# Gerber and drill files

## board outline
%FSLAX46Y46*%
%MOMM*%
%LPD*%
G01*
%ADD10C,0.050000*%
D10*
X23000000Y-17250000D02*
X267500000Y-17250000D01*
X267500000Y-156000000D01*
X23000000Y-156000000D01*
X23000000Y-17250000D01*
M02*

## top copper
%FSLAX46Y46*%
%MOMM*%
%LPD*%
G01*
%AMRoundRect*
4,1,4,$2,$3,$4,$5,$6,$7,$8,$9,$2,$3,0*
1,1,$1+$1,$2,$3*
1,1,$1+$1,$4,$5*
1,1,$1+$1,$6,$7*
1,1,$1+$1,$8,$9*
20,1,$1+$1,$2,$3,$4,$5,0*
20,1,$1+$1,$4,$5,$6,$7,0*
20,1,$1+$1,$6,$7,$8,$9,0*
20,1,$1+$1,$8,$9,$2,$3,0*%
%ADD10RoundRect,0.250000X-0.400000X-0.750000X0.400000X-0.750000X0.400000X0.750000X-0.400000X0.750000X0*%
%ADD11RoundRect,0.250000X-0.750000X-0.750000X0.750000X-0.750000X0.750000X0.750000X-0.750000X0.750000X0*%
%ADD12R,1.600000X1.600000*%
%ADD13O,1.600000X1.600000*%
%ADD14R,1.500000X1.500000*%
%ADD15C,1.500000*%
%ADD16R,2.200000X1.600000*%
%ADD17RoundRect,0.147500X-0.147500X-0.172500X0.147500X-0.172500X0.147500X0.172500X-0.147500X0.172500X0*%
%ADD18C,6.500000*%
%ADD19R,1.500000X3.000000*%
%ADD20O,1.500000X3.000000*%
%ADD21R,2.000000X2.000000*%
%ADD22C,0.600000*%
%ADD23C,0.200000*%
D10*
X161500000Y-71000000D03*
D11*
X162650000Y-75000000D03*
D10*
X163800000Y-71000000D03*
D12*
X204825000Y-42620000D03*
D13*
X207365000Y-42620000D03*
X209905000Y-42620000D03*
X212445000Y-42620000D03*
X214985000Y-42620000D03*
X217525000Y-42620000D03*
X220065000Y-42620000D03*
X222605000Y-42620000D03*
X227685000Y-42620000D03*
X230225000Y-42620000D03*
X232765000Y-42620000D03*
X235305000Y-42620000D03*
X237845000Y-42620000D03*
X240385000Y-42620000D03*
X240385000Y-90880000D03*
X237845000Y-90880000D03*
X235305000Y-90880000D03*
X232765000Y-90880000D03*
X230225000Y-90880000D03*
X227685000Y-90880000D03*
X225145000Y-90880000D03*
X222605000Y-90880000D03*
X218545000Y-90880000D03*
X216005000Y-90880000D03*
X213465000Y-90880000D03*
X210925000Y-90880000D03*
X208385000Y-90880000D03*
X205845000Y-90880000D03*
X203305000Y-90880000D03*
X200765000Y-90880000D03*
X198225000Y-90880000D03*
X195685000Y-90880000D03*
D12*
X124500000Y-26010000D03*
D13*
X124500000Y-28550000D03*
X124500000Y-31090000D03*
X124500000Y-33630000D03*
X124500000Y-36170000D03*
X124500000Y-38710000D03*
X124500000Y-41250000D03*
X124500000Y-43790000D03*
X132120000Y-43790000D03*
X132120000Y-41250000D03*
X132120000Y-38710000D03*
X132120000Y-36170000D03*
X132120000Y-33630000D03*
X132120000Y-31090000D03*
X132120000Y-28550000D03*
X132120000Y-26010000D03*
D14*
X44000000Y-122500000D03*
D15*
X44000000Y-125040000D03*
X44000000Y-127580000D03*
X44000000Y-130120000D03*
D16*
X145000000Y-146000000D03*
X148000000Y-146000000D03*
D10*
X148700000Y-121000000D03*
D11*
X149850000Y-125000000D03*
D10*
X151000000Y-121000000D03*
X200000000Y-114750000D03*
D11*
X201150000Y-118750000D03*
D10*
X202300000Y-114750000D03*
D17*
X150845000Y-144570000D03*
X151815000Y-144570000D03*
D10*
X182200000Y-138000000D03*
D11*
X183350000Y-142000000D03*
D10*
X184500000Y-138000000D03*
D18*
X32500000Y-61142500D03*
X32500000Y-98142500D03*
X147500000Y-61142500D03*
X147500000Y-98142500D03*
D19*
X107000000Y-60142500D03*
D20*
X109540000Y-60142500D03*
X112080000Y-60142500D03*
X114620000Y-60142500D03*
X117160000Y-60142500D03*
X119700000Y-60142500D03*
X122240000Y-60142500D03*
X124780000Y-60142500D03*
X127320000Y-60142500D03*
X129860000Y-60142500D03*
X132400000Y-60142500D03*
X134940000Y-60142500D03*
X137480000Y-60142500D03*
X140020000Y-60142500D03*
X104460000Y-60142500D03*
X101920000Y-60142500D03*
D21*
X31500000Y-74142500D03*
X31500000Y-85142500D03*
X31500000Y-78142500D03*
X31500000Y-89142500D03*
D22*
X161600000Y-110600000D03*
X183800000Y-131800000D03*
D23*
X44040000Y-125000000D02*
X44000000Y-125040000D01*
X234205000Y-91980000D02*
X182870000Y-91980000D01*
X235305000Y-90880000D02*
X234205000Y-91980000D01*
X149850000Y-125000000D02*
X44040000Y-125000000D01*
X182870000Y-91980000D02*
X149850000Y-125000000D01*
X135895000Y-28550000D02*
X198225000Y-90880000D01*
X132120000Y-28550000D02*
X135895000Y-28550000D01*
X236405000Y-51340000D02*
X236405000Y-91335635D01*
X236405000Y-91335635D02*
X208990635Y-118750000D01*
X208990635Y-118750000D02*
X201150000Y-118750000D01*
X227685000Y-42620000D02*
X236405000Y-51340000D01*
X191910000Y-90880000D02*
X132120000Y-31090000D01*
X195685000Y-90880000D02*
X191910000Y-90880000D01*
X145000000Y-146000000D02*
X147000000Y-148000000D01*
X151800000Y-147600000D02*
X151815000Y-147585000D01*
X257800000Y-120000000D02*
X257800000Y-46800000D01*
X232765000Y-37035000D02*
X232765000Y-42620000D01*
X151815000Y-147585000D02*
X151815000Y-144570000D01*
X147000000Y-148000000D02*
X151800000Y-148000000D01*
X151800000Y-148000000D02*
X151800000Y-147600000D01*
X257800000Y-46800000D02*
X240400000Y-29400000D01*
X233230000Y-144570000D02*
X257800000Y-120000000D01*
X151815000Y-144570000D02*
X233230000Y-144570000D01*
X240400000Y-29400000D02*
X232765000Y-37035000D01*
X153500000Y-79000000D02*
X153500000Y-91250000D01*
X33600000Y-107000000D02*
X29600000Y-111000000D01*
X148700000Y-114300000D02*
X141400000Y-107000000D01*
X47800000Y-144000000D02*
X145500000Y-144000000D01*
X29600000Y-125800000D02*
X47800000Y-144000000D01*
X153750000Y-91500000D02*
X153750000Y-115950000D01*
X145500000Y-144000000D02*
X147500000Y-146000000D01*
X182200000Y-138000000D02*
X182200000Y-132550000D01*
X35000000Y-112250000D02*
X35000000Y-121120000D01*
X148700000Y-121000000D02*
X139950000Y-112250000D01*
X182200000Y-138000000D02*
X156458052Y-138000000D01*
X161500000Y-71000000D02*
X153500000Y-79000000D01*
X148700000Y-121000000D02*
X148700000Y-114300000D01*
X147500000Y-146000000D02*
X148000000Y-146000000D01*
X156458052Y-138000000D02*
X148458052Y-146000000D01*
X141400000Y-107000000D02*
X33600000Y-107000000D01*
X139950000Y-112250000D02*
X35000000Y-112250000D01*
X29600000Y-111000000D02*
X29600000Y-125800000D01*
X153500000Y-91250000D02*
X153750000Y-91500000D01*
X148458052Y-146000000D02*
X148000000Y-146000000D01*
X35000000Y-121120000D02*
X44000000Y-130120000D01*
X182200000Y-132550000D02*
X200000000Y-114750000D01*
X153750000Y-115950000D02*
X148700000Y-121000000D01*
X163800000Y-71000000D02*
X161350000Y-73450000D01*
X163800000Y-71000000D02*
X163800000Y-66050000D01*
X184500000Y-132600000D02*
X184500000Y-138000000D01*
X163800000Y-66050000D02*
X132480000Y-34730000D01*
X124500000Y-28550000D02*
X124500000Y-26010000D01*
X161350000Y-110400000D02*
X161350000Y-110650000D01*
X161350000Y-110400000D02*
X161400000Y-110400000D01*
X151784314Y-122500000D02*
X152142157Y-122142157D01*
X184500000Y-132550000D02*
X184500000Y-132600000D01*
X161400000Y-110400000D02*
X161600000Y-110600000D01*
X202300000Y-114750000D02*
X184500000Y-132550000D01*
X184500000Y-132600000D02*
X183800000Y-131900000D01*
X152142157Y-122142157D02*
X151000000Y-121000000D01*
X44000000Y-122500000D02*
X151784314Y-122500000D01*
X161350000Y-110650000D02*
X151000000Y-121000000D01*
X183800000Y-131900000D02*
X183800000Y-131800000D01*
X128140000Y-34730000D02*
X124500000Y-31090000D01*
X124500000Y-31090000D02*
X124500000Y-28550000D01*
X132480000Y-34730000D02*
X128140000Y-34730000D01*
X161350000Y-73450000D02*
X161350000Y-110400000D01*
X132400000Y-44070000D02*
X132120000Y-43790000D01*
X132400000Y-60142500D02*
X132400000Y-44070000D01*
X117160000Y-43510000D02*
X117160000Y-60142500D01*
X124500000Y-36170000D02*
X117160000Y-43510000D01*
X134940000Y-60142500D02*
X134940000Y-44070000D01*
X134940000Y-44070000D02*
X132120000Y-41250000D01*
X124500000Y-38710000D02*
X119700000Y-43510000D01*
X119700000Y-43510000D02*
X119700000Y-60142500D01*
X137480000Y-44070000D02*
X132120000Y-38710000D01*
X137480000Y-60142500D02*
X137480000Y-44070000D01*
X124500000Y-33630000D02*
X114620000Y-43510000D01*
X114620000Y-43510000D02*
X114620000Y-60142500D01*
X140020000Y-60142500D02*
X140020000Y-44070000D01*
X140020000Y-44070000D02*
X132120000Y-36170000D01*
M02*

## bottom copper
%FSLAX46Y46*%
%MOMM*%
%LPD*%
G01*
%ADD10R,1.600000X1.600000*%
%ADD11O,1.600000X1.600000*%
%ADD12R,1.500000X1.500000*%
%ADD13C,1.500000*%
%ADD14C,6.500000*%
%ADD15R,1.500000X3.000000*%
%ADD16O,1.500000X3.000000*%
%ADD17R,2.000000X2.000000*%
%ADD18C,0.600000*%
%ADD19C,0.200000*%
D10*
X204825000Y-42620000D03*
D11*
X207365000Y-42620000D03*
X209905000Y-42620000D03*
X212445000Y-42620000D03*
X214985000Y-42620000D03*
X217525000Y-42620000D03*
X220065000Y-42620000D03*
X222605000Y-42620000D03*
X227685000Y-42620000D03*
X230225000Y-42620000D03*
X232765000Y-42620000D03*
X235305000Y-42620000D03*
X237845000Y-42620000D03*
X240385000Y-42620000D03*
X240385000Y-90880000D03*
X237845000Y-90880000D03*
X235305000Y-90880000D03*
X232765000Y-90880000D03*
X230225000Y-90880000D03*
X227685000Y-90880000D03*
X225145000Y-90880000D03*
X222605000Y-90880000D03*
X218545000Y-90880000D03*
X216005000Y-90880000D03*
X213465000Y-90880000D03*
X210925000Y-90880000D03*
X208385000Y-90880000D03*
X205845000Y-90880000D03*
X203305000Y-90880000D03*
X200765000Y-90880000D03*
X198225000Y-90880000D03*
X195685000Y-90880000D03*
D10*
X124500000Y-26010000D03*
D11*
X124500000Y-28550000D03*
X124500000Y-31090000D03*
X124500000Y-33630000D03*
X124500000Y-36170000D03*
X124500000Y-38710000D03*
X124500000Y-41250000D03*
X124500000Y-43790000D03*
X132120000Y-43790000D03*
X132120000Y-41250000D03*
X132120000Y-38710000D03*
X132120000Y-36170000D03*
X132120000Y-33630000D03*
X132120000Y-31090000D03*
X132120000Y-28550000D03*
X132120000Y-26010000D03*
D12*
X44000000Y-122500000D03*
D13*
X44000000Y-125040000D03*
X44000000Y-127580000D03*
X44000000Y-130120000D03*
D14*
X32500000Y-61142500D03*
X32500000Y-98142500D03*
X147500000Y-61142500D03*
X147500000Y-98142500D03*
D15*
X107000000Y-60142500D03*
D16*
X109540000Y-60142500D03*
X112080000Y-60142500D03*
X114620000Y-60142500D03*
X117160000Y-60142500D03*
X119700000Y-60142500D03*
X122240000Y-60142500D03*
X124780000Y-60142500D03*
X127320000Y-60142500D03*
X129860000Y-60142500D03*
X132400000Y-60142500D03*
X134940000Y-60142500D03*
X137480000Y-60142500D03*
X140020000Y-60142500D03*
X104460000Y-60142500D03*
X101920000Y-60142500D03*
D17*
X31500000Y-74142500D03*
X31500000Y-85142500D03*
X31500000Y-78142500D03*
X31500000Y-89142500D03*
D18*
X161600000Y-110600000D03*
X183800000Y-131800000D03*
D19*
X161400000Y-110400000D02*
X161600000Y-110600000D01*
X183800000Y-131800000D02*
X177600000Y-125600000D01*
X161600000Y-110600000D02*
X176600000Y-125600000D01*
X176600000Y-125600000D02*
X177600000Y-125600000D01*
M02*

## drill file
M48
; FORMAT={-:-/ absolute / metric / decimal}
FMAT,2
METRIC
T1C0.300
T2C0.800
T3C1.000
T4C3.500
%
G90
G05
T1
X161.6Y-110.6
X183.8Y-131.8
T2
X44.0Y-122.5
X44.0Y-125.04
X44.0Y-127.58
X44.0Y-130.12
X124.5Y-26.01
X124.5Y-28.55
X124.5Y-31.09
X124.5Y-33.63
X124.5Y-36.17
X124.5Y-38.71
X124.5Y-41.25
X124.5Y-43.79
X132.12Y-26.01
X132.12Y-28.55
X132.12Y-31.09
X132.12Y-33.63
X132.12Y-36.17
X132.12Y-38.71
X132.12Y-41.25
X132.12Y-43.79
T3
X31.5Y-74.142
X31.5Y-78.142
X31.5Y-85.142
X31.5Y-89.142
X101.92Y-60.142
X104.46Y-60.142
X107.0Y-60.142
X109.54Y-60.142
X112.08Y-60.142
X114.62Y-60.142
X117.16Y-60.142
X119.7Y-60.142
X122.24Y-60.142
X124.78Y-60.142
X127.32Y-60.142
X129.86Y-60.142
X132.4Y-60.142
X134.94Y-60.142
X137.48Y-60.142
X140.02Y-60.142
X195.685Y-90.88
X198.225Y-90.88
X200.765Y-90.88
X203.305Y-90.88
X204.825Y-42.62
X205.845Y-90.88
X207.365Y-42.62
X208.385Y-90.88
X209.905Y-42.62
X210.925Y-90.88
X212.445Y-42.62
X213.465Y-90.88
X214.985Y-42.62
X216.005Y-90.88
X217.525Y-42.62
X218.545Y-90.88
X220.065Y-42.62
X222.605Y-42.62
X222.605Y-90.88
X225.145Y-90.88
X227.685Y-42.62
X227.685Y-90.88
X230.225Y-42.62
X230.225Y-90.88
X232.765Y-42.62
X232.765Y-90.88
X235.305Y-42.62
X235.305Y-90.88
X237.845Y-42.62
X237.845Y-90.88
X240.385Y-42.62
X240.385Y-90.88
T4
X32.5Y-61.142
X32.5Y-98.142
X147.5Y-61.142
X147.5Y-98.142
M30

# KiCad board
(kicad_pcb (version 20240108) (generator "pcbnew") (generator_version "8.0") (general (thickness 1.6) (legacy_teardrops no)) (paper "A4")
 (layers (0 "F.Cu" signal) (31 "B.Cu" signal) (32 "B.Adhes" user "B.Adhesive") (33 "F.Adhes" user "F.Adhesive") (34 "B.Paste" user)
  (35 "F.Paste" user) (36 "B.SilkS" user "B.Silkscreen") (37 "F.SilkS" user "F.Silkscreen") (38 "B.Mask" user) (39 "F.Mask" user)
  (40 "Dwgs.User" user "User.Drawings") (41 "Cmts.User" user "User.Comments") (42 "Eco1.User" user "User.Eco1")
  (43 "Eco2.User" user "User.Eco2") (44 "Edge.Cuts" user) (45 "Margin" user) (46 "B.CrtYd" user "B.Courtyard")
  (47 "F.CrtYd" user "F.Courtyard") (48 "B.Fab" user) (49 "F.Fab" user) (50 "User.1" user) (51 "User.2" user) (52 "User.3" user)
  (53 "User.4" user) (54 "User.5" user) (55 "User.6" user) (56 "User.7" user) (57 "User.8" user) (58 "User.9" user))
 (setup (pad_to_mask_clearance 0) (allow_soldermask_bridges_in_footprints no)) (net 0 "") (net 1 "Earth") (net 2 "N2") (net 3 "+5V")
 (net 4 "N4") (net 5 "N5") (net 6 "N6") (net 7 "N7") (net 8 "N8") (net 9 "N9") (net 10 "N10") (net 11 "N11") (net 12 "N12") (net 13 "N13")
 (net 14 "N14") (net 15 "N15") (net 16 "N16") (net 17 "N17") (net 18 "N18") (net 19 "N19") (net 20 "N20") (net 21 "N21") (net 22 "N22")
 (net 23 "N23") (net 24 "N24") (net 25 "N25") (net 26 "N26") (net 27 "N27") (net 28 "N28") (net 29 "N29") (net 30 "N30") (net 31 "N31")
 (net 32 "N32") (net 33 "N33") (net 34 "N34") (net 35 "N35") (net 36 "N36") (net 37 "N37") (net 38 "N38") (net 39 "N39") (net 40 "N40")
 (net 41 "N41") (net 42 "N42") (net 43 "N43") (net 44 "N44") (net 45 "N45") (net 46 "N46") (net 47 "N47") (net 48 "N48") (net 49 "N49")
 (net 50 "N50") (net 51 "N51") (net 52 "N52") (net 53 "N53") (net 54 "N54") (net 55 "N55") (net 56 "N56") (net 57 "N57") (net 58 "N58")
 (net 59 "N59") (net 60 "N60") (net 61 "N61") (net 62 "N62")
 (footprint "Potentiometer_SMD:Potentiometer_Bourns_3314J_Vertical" (layer "F.Cu") (at 162.65 73)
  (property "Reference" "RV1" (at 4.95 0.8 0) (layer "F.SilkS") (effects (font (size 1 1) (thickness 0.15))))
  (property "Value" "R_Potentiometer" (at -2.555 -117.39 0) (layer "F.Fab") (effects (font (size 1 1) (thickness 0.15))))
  (pad "1" smd roundrect (at -1.15 -2) (size 1.3 2) (layers "F.Cu" "F.Paste" "F.Mask") (roundrect_rratio 0.1923076923) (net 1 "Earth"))
  (pad "2" smd roundrect (at 0 2) (size 2 2) (layers "F.Cu" "F.Paste" "F.Mask") (roundrect_rratio 0.125) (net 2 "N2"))
  (pad "3" smd roundrect (at 1.15 -2) (size 1.3 2) (layers "F.Cu" "F.Paste" "F.Mask") (roundrect_rratio 0.1923076923) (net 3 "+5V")))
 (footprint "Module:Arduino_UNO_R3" (layer "F.Cu") (at 204.825 42.62)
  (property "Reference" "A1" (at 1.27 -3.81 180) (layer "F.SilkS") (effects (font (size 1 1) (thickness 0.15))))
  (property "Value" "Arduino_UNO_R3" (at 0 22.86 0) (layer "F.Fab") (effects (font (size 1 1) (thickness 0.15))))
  (pad "1" thru_hole rect (at 0 0 90) (size 1.6 1.6) (drill 1) (layers "*.Cu" "*.Mask") (remove_unused_layers no) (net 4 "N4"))
  (pad "2" thru_hole oval (at 2.54 0 90) (size 1.6 1.6) (drill 1) (layers "*.Cu" "*.Mask") (remove_unused_layers no) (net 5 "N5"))
  (pad "3" thru_hole oval (at 5.08 0 90) (size 1.6 1.6) (drill 1) (layers "*.Cu" "*.Mask") (remove_unused_layers no) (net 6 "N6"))
  (pad "4" thru_hole oval (at 7.62 0 90) (size 1.6 1.6) (drill 1) (layers "*.Cu" "*.Mask") (remove_unused_layers no) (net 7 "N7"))
  (pad "5" thru_hole oval (at 10.16 0 90) (size 1.6 1.6) (drill 1) (layers "*.Cu" "*.Mask") (remove_unused_layers no) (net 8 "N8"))
  (pad "6" thru_hole oval (at 12.7 0 90) (size 1.6 1.6) (drill 1) (layers "*.Cu" "*.Mask") (remove_unused_layers no) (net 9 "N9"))
  (pad "7" thru_hole oval (at 15.24 0 90) (size 1.6 1.6) (drill 1) (layers "*.Cu" "*.Mask") (remove_unused_layers no) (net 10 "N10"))
  (pad "8" thru_hole oval (at 17.78 0 90) (size 1.6 1.6) (drill 1) (layers "*.Cu" "*.Mask") (remove_unused_layers no) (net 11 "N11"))
  (pad "9" thru_hole oval (at 22.86 0 90) (size 1.6 1.6) (drill 1) (layers "*.Cu" "*.Mask") (remove_unused_layers no) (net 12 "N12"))
  (pad "10" thru_hole oval (at 25.4 0 90) (size 1.6 1.6) (drill 1) (layers "*.Cu" "*.Mask") (remove_unused_layers no) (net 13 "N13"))
  (pad "11" thru_hole oval (at 27.94 0 90) (size 1.6 1.6) (drill 1) (layers "*.Cu" "*.Mask") (remove_unused_layers no) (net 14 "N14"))
  (pad "12" thru_hole oval (at 30.48 0 90) (size 1.6 1.6) (drill 1) (layers "*.Cu" "*.Mask") (remove_unused_layers no) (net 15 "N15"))
  (pad "13" thru_hole oval (at 33.02 0 90) (size 1.6 1.6) (drill 1) (layers "*.Cu" "*.Mask") (remove_unused_layers no) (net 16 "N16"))
  (pad "14" thru_hole oval (at 35.56 0 90) (size 1.6 1.6) (drill 1) (layers "*.Cu" "*.Mask") (remove_unused_layers no) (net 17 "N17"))
  (pad "15" thru_hole oval (at 35.56 48.26 90) (size 1.6 1.6) (drill 1) (layers "*.Cu" "*.Mask") (remove_unused_layers no) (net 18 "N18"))
  (pad "16" thru_hole oval (at 33.02 48.26 90) (size 1.6 1.6) (drill 1) (layers "*.Cu" "*.Mask") (remove_unused_layers no) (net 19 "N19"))
  (pad "17" thru_hole oval (at 30.48 48.26 90) (size 1.6 1.6) (drill 1) (layers "*.Cu" "*.Mask") (remove_unused_layers no) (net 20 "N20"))
  (pad "18" thru_hole oval (at 27.94 48.26 90) (size 1.6 1.6) (drill 1) (layers "*.Cu" "*.Mask") (remove_unused_layers no) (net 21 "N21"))
  (pad "19" thru_hole oval (at 25.4 48.26 90) (size 1.6 1.6) (drill 1) (layers "*.Cu" "*.Mask") (remove_unused_layers no) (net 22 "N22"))
  (pad "20" thru_hole oval (at 22.86 48.26 90) (size 1.6 1.6) (drill 1) (layers "*.Cu" "*.Mask") (remove_unused_layers no) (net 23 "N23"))
  (pad "21" thru_hole oval (at 20.32 48.26 90) (size 1.6 1.6) (drill 1) (layers "*.Cu" "*.Mask") (remove_unused_layers no) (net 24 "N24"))
  (pad "22" thru_hole oval (at 17.78 48.26 90) (size 1.6 1.6) (drill 1) (layers "*.Cu" "*.Mask") (remove_unused_layers no) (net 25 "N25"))
  (pad "23" thru_hole oval (at 13.72 48.26 90) (size 1.6 1.6) (drill 1) (layers "*.Cu" "*.Mask") (remove_unused_layers no) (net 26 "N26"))
  (pad "24" thru_hole oval (at 11.18 48.26 90) (size 1.6 1.6) (drill 1) (layers "*.Cu" "*.Mask") (remove_unused_layers no) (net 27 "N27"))
  (pad "25" thru_hole oval (at 8.64 48.26 90) (size 1.6 1.6) (drill 1) (layers "*.Cu" "*.Mask") (remove_unused_layers no) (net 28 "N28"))
  (pad "26" thru_hole oval (at 6.1 48.26 90) (size 1.6 1.6) (drill 1) (layers "*.Cu" "*.Mask") (remove_unused_layers no) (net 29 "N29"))
  (pad "27" thru_hole oval (at 3.56 48.26 90) (size 1.6 1.6) (drill 1) (layers "*.Cu" "*.Mask") (remove_unused_layers no) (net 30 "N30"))
  (pad "28" thru_hole oval (at 1.02 48.26 90) (size 1.6 1.6) (drill 1) (layers "*.Cu" "*.Mask") (remove_unused_layers no) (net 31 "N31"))
  (pad "29" thru_hole oval (at -1.52 48.26 90) (size 1.6 1.6) (drill 1) (layers "*.Cu" "*.Mask") (remove_unused_layers no) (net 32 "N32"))
  (pad "30" thru_hole oval (at -4.06 48.26 90) (size 1.6 1.6) (drill 1) (layers "*.Cu" "*.Mask") (remove_unused_layers no) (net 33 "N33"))
  (pad "31" thru_hole oval (at -6.6 48.26 90) (size 1.6 1.6) (drill 1) (layers "*.Cu" "*.Mask") (remove_unused_layers no) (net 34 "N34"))
  (pad "32" thru_hole oval (at -9.14 48.26 90) (size 1.6 1.6) (drill 1) (layers "*.Cu" "*.Mask") (remove_unused_layers no) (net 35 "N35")))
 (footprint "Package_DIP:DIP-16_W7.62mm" (layer "F.Cu") (at 124.5 26.01)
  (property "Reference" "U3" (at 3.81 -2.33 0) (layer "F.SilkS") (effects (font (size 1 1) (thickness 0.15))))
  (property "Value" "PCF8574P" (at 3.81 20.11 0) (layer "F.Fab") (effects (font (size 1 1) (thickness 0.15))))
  (pad "1" thru_hole rect (at 0 0) (size 1.6 1.6) (drill 0.8) (layers "*.Cu" "*.Mask") (remove_unused_layers no) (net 3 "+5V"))
  (pad "2" thru_hole oval (at 0 2.54) (size 1.6 1.6) (drill 0.8) (layers "*.Cu" "*.Mask") (remove_unused_layers no) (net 3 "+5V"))
  (pad "3" thru_hole oval (at 0 5.08) (size 1.6 1.6) (drill 0.8) (layers "*.Cu" "*.Mask") (remove_unused_layers no) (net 3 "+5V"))
  (pad "4" thru_hole oval (at 0 7.62) (size 1.6 1.6) (drill 0.8) (layers "*.Cu" "*.Mask") (remove_unused_layers no) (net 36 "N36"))
  (pad "5" thru_hole oval (at 0 10.16) (size 1.6 1.6) (drill 0.8) (layers "*.Cu" "*.Mask") (remove_unused_layers no) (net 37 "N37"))
  (pad "6" thru_hole oval (at 0 12.7) (size 1.6 1.6) (drill 0.8) (layers "*.Cu" "*.Mask") (remove_unused_layers no) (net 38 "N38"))
  (pad "7" thru_hole oval (at 0 15.24) (size 1.6 1.6) (drill 0.8) (layers "*.Cu" "*.Mask") (remove_unused_layers no) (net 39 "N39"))
  (pad "8" thru_hole oval (at 0 17.78) (size 1.6 1.6) (drill 0.8) (layers "*.Cu" "*.Mask") (remove_unused_layers no) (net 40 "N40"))
  (pad "9" thru_hole oval (at 7.62 17.78) (size 1.6 1.6) (drill 0.8) (layers "*.Cu" "*.Mask") (remove_unused_layers no) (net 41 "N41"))
  (pad "10" thru_hole oval (at 7.62 15.24) (size 1.6 1.6) (drill 0.8) (layers "*.Cu" "*.Mask") (remove_unused_layers no) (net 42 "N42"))
  (pad "11" thru_hole oval (at 7.62 12.7) (size 1.6 1.6) (drill 0.8) (layers "*.Cu" "*.Mask") (remove_unused_layers no) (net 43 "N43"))
  (pad "12" thru_hole oval (at 7.62 10.16) (size 1.6 1.6) (drill 0.8) (layers "*.Cu" "*.Mask") (remove_unused_layers no) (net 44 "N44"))
  (pad "13" thru_hole oval (at 7.62 7.62) (size 1.6 1.6) (drill 0.8) (layers "*.Cu" "*.Mask") (remove_unused_layers no) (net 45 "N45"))
  (pad "14" thru_hole oval (at 7.62 5.08) (size 1.6 1.6) (drill 0.8) (layers "*.Cu" "*.Mask") (remove_unused_layers no) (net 35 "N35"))
  (pad "15" thru_hole oval (at 7.62 2.54) (size 1.6 1.6) (drill 0.8) (layers "*.Cu" "*.Mask") (remove_unused_layers no) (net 34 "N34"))
  (pad "16" thru_hole oval (at 7.62 0) (size 1.6 1.6) (drill 0.8) (layers "*.Cu" "*.Mask") (remove_unused_layers no) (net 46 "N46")))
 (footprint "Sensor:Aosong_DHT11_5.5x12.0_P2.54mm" (layer "F.Cu") (at 44 122.5)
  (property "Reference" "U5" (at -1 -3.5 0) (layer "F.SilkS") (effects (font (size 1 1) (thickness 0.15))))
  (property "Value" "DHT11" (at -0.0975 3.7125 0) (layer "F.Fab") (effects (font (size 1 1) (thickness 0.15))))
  (pad "1" thru_hole rect (at 0 0) (size 1.5 1.5) (drill 0.8) (layers "*.Cu" "*.Mask") (remove_unused_layers no) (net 3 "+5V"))
  (pad "2" thru_hole circle (at 0 2.54) (size 1.5 1.5) (drill 0.8) (layers "*.Cu" "*.Mask") (remove_unused_layers no) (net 20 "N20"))
  (pad "3" thru_hole circle (at 0 5.08) (size 1.5 1.5) (drill 0.8) (layers "*.Cu" "*.Mask") (remove_unused_layers no) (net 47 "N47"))
  (pad "4" thru_hole circle (at 0 7.62) (size 1.5 1.5) (drill 0.8) (layers "*.Cu" "*.Mask") (remove_unused_layers no) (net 1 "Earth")))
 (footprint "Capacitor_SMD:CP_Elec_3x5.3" (layer "F.Cu") (at 146.5 146)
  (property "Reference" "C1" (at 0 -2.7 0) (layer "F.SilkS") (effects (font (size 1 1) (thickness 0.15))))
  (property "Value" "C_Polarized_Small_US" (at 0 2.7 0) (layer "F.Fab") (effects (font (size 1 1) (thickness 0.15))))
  (pad "1" smd rect (at -1.5 0) (size 2.2 1.6) (layers "F.Cu" "F.Paste" "F.Mask") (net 14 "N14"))
  (pad "2" smd rect (at 1.5 0) (size 2.2 1.6) (layers "F.Cu" "F.Paste" "F.Mask") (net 1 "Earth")))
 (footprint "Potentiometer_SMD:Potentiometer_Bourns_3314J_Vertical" (layer "F.Cu") (at 149.85 123)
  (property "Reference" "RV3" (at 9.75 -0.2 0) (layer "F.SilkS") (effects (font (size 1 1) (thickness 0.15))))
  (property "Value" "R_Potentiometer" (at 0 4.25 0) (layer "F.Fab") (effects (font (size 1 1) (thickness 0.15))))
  (pad "1" smd roundrect (at -1.15 -2) (size 1.3 2) (layers "F.Cu" "F.Paste" "F.Mask") (roundrect_rratio 0.1923076923) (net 1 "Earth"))
  (pad "2" smd roundrect (at 0 2) (size 2 2) (layers "F.Cu" "F.Paste" "F.Mask") (roundrect_rratio 0.125) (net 20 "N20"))
  (pad "3" smd roundrect (at 1.15 -2) (size 1.3 2) (layers "F.Cu" "F.Paste" "F.Mask") (roundrect_rratio 0.1923076923) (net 3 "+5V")))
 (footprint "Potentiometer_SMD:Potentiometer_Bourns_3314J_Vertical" (layer "F.Cu") (at 201.15 116.75)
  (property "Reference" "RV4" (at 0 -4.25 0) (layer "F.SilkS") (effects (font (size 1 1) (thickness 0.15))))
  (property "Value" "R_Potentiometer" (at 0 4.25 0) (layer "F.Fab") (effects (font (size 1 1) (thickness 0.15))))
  (pad "1" smd roundrect (at -1.15 -2) (size 1.3 2) (layers "F.Cu" "F.Paste" "F.Mask") (roundrect_rratio 0.1923076923) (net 1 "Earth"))
  (pad "2" smd roundrect (at 0 2) (size 2 2) (layers "F.Cu" "F.Paste" "F.Mask") (roundrect_rratio 0.125) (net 12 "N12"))
  (pad "3" smd roundrect (at 1.15 -2) (size 1.3 2) (layers "F.Cu" "F.Paste" "F.Mask") (roundrect_rratio 0.1923076923) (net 3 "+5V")))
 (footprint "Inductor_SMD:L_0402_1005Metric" (layer "F.Cu") (at 151.33 144.57)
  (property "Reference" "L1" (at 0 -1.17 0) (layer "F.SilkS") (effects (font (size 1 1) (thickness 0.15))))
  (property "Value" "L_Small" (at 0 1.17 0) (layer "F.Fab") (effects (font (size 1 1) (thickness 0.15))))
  (pad "1" smd roundrect (at -0.485 0) (size 0.59 0.64) (layers "F.Cu" "F.Paste" "F.Mask") (roundrect_rratio 0.25) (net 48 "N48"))
  (pad "2" smd roundrect (at 0.485 0) (size 0.59 0.64) (layers "F.Cu" "F.Paste" "F.Mask") (roundrect_rratio 0.25) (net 14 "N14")))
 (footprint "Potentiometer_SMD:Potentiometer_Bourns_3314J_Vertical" (layer "F.Cu") (at 183.35 140)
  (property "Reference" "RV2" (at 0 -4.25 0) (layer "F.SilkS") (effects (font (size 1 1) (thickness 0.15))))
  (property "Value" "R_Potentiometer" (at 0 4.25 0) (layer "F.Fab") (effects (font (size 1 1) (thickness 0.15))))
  (pad "1" smd roundrect (at -1.15 -2) (size 1.3 2) (layers "F.Cu" "F.Paste" "F.Mask") (roundrect_rratio 0.1923076923) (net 1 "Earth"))
  (pad "2" smd roundrect (at 0 2) (size 2 2) (layers "F.Cu" "F.Paste" "F.Mask") (roundrect_rratio 0.125) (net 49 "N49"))
  (pad "3" smd roundrect (at 1.15 -2) (size 1.3 2) (layers "F.Cu" "F.Paste" "F.Mask") (roundrect_rratio 0.1923076923) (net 3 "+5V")))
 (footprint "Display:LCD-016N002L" (layer "F.Cu") (at 107 60.1425)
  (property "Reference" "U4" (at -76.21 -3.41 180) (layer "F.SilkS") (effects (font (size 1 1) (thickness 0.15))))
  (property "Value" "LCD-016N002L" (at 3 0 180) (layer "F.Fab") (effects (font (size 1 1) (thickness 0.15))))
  (pad "" thru_hole circle (at -74.5 1 180) (size 6.5 6.5) (drill 3.5) (layers "*.Cu" "*.Mask") (remove_unused_layers no))
  (pad "" thru_hole circle (at -74.5 38 180) (size 6.5 6.5) (drill 3.5) (layers "*.Cu" "*.Mask") (remove_unused_layers no))
  (pad "" thru_hole circle (at 40.5 1 180) (size 6.5 6.5) (drill 3.5) (layers "*.Cu" "*.Mask") (remove_unused_layers no))
  (pad "" thru_hole circle (at 40.5 38 180) (size 6.5 6.5) (drill 3.5) (layers "*.Cu" "*.Mask") (remove_unused_layers no))
  (pad "1" thru_hole rect (at 0 0 180) (size 1.5 3) (drill 1) (layers "*.Cu" "*.Mask") (remove_unused_layers no) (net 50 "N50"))
  (pad "2" thru_hole oval (at 2.54 0 180) (size 1.5 3) (drill 1) (layers "*.Cu" "*.Mask") (remove_unused_layers no) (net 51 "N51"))
  (pad "3" thru_hole oval (at 5.08 0 180) (size 1.5 3) (drill 1) (layers "*.Cu" "*.Mask") (remove_unused_layers no) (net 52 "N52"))
  (pad "4" thru_hole oval (at 7.62 0 180) (size 1.5 3) (drill 1) (layers "*.Cu" "*.Mask") (remove_unused_layers no) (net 36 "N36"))
  (pad "5" thru_hole oval (at 10.16 0 180) (size 1.5 3) (drill 1) (layers "*.Cu" "*.Mask") (remove_unused_layers no) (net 37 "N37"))
  (pad "6" thru_hole oval (at 12.7 0 180) (size 1.5 3) (drill 1) (layers "*.Cu" "*.Mask") (remove_unused_layers no) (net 38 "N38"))
  (pad "7" thru_hole oval (at 15.24 0 180) (size 1.5 3) (drill 1) (layers "*.Cu" "*.Mask") (remove_unused_layers no) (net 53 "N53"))
  (pad "8" thru_hole oval (at 17.78 0 180) (size 1.5 3) (drill 1) (layers "*.Cu" "*.Mask") (remove_unused_layers no) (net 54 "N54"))
  (pad "9" thru_hole oval (at 20.32 0 180) (size 1.5 3) (drill 1) (layers "*.Cu" "*.Mask") (remove_unused_layers no) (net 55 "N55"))
  (pad "10" thru_hole oval (at 22.86 0 180) (size 1.5 3) (drill 1) (layers "*.Cu" "*.Mask") (remove_unused_layers no) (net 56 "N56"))
  (pad "11" thru_hole oval (at 25.4 0 180) (size 1.5 3) (drill 1) (layers "*.Cu" "*.Mask") (remove_unused_layers no) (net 41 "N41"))
  (pad "12" thru_hole oval (at 27.94 0 180) (size 1.5 3) (drill 1) (layers "*.Cu" "*.Mask") (remove_unused_layers no) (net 42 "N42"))
  (pad "13" thru_hole oval (at 30.48 0 180) (size 1.5 3) (drill 1) (layers "*.Cu" "*.Mask") (remove_unused_layers no) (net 43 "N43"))
  (pad "14" thru_hole oval (at 33.02 0 180) (size 1.5 3) (drill 1) (layers "*.Cu" "*.Mask") (remove_unused_layers no) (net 44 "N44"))
  (pad "15" thru_hole oval (at -2.54 0 180) (size 1.5 3) (drill 1) (layers "*.Cu" "*.Mask") (remove_unused_layers no) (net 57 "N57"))
  (pad "16" thru_hole oval (at -5.08 0 180) (size 1.5 3) (drill 1) (layers "*.Cu" "*.Mask") (remove_unused_layers no) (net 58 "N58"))
  (pad "A1" thru_hole rect (at -75.5 14 180) (size 2 2) (drill 1) (layers "*.Cu" "*.Mask") (remove_unused_layers no) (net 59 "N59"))
  (pad "A2" thru_hole rect (at -75.5 25 180) (size 2 2) (drill 1) (layers "*.Cu" "*.Mask") (remove_unused_layers no) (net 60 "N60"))
  (pad "K1" thru_hole rect (at -75.5 18 180) (size 2 2) (drill 1) (layers "*.Cu" "*.Mask") (remove_unused_layers no) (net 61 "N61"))
  (pad "K2" thru_hole rect (at -75.5 29 180) (size 2 2) (drill 1) (layers "*.Cu" "*.Mask") (remove_unused_layers no) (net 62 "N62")))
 (gr_rect (start 23 17.25) (end 267.5 156) (stroke (width 0.05) (type default)) (fill none) (layer "Edge.Cuts"))
 (segment (start 44.04 125) (end 44 125.04) (width 0.2) (layer "F.Cu") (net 20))
 (segment (start 234.205 91.98) (end 182.87 91.98) (width 0.2) (layer "F.Cu") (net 20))
 (segment (start 235.305 90.88) (end 234.205 91.98) (width 0.2) (layer "F.Cu") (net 20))
 (segment (start 149.85 125) (end 44.04 125) (width 0.2) (layer "F.Cu") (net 20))
 (segment (start 182.87 91.98) (end 149.85 125) (width 0.2) (layer "F.Cu") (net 20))
 (segment (start 135.895 28.55) (end 198.225 90.88) (width 0.2) (layer "F.Cu") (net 34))
 (segment (start 132.12 28.55) (end 135.895 28.55) (width 0.2) (layer "F.Cu") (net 34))
 (segment (start 236.405 51.34) (end 236.405 91.335635) (width 0.2) (layer "F.Cu") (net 12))
 (segment (start 236.405 91.335635) (end 208.990635 118.75) (width 0.2) (layer "F.Cu") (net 12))
 (segment (start 208.990635 118.75) (end 201.15 118.75) (width 0.2) (layer "F.Cu") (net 12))
 (segment (start 227.685 42.62) (end 236.405 51.34) (width 0.2) (layer "F.Cu") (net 12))
 (segment (start 191.91 90.88) (end 132.12 31.09) (width 0.2) (layer "F.Cu") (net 35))
 (segment (start 195.685 90.88) (end 191.91 90.88) (width 0.2) (layer "F.Cu") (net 35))
 (segment (start 145 146) (end 147 148) (width 0.2) (layer "F.Cu") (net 14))
 (segment (start 151.8 147.6) (end 151.815 147.585) (width 0.2) (layer "F.Cu") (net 14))
 (segment (start 257.8 120) (end 257.8 46.8) (width 0.2) (layer "F.Cu") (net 14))
 (segment (start 232.765 37.035) (end 232.765 42.62) (width 0.2) (layer "F.Cu") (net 14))
 (segment (start 151.815 147.585) (end 151.815 144.57) (width 0.2) (layer "F.Cu") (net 14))
 (segment (start 147 148) (end 151.8 148) (width 0.2) (layer "F.Cu") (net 14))
 (segment (start 151.8 148) (end 151.8 147.6) (width 0.2) (layer "F.Cu") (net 14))
 (segment (start 257.8 46.8) (end 240.4 29.4) (width 0.2) (layer "F.Cu") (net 14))
 (segment (start 233.23 144.57) (end 257.8 120) (width 0.2) (layer "F.Cu") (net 14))
 (segment (start 151.815 144.57) (end 233.23 144.57) (width 0.2) (layer "F.Cu") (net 14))
 (segment (start 240.4 29.4) (end 232.765 37.035) (width 0.2) (layer "F.Cu") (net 14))
 (segment (start 153.5 79) (end 153.5 91.25) (width 0.2) (layer "F.Cu") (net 1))
 (segment (start 33.6 107) (end 29.6 111) (width 0.2) (layer "F.Cu") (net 1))
 (segment (start 148.7 114.3) (end 141.4 107) (width 0.2) (layer "F.Cu") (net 1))
 (segment (start 47.8 144) (end 145.5 144) (width 0.2) (layer "F.Cu") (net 1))
 (segment (start 29.6 125.8) (end 47.8 144) (width 0.2) (layer "F.Cu") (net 1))
 (segment (start 153.75 91.5) (end 153.75 115.95) (width 0.2) (layer "F.Cu") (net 1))
 (segment (start 145.5 144) (end 147.5 146) (width 0.2) (layer "F.Cu") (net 1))
 (segment (start 182.2 138) (end 182.2 132.55) (width 0.2) (layer "F.Cu") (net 1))
 (segment (start 35 112.25) (end 35 121.12) (width 0.2) (layer "F.Cu") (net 1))
 (segment (start 148.7 121) (end 139.95 112.25) (width 0.2) (layer "F.Cu") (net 1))
 (segment (start 182.2 138) (end 156.458052 138) (width 0.2) (layer "F.Cu") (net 1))
 (segment (start 161.5 71) (end 153.5 79) (width 0.2) (layer "F.Cu") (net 1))
 (segment (start 148.7 121) (end 148.7 114.3) (width 0.2) (layer "F.Cu") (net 1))
 (segment (start 147.5 146) (end 148 146) (width 0.2) (layer "F.Cu") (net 1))
 (segment (start 156.458052 138) (end 148.458052 146) (width 0.2) (layer "F.Cu") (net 1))
 (segment (start 141.4 107) (end 33.6 107) (width 0.2) (layer "F.Cu") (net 1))
 (segment (start 139.95 112.25) (end 35 112.25) (width 0.2) (layer "F.Cu") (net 1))
 (segment (start 29.6 111) (end 29.6 125.8) (width 0.2) (layer "F.Cu") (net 1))
 (segment (start 153.5 91.25) (end 153.75 91.5) (width 0.2) (layer "F.Cu") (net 1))
 (segment (start 148.458052 146) (end 148 146) (width 0.2) (layer "F.Cu") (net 1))
 (segment (start 35 121.12) (end 44 130.12) (width 0.2) (layer "F.Cu") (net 1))
 (segment (start 182.2 132.55) (end 200 114.75) (width 0.2) (layer "F.Cu") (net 1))
 (segment (start 153.75 115.95) (end 148.7 121) (width 0.2) (layer "F.Cu") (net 1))
 (segment (start 163.8 71) (end 161.35 73.45) (width 0.2) (layer "F.Cu") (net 3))
 (segment (start 163.8 71) (end 163.8 66.05) (width 0.2) (layer "F.Cu") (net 3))
 (segment (start 184.5 132.6) (end 184.5 138) (width 0.2) (layer "F.Cu") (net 3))
 (segment (start 163.8 66.05) (end 132.48 34.73) (width 0.2) (layer "F.Cu") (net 3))
 (segment (start 124.5 28.55) (end 124.5 26.01) (width 0.2) (layer "F.Cu") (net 3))
 (segment (start 161.35 110.4) (end 161.35 110.65) (width 0.2) (layer "F.Cu") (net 3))
 (segment (start 161.35 110.4) (end 161.4 110.4) (width 0.2) (layer "F.Cu") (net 3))
 (segment (start 151.784314 122.5) (end 152.142157 122.142157) (width 0.2) (layer "F.Cu") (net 3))
 (segment (start 184.5 132.55) (end 184.5 132.6) (width 0.2) (layer "F.Cu") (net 3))
 (segment (start 161.4 110.4) (end 161.6 110.6) (width 0.2) (layer "F.Cu") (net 3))
 (segment (start 202.3 114.75) (end 184.5 132.55) (width 0.2) (layer "F.Cu") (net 3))
 (segment (start 184.5 132.6) (end 183.8 131.9) (width 0.2) (layer "F.Cu") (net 3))
 (segment (start 152.142157 122.142157) (end 151 121) (width 0.2) (layer "F.Cu") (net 3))
 (segment (start 44 122.5) (end 151.784314 122.5) (width 0.2) (layer "F.Cu") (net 3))
 (segment (start 161.35 110.65) (end 151 121) (width 0.2) (layer "F.Cu") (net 3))
 (segment (start 183.8 131.9) (end 183.8 131.8) (width 0.2) (layer "F.Cu") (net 3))
 (segment (start 128.14 34.73) (end 124.5 31.09) (width 0.2) (layer "F.Cu") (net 3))
 (segment (start 124.5 31.09) (end 124.5 28.55) (width 0.2) (layer "F.Cu") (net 3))
 (segment (start 132.48 34.73) (end 128.14 34.73) (width 0.2) (layer "F.Cu") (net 3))
 (segment (start 161.35 73.45) (end 161.35 110.4) (width 0.2) (layer "F.Cu") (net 3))
 (via (at 161.6 110.6) (size 0.6) (drill 0.3) (layers "F.Cu" "B.Cu") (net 3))
 (via (at 183.8 131.8) (size 0.6) (drill 0.3) (layers "F.Cu" "B.Cu") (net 3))
 (segment (start 161.4 110.4) (end 161.6 110.6) (width 0.2) (layer "B.Cu") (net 3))
 (segment (start 183.8 131.8) (end 177.6 125.6) (width 0.2) (layer "B.Cu") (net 3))
 (segment (start 161.6 110.6) (end 176.6 125.6) (width 0.2) (layer "B.Cu") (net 3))
 (segment (start 176.6 125.6) (end 177.6 125.6) (width 0.2) (layer "B.Cu") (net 3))
 (segment (start 132.4 44.07) (end 132.12 43.79) (width 0.2) (layer "F.Cu") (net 41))
 (segment (start 132.4 60.1425) (end 132.4 44.07) (width 0.2) (layer "F.Cu") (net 41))
 (segment (start 117.16 43.51) (end 117.16 60.1425) (width 0.2) (layer "F.Cu") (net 37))
 (segment (start 124.5 36.17) (end 117.16 43.51) (width 0.2) (layer "F.Cu") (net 37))
 (segment (start 134.94 60.1425) (end 134.94 44.07) (width 0.2) (layer "F.Cu") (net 42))
 (segment (start 134.94 44.07) (end 132.12 41.25) (width 0.2) (layer "F.Cu") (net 42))
 (segment (start 124.5 38.71) (end 119.7 43.51) (width 0.2) (layer "F.Cu") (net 38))
 (segment (start 119.7 43.51) (end 119.7 60.1425) (width 0.2) (layer "F.Cu") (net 38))
 (segment (start 137.48 44.07) (end 132.12 38.71) (width 0.2) (layer "F.Cu") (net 43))
 (segment (start 137.48 60.1425) (end 137.48 44.07) (width 0.2) (layer "F.Cu") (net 43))
 (segment (start 124.5 33.63) (end 114.62 43.51) (width 0.2) (layer "F.Cu") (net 36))
 (segment (start 114.62 43.51) (end 114.62 60.1425) (width 0.2) (layer "F.Cu") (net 36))
 (segment (start 140.02 60.1425) (end 140.02 44.07) (width 0.2) (layer "F.Cu") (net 44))
 (segment (start 140.02 44.07) (end 132.12 36.17) (width 0.2) (layer "F.Cu") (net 44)))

